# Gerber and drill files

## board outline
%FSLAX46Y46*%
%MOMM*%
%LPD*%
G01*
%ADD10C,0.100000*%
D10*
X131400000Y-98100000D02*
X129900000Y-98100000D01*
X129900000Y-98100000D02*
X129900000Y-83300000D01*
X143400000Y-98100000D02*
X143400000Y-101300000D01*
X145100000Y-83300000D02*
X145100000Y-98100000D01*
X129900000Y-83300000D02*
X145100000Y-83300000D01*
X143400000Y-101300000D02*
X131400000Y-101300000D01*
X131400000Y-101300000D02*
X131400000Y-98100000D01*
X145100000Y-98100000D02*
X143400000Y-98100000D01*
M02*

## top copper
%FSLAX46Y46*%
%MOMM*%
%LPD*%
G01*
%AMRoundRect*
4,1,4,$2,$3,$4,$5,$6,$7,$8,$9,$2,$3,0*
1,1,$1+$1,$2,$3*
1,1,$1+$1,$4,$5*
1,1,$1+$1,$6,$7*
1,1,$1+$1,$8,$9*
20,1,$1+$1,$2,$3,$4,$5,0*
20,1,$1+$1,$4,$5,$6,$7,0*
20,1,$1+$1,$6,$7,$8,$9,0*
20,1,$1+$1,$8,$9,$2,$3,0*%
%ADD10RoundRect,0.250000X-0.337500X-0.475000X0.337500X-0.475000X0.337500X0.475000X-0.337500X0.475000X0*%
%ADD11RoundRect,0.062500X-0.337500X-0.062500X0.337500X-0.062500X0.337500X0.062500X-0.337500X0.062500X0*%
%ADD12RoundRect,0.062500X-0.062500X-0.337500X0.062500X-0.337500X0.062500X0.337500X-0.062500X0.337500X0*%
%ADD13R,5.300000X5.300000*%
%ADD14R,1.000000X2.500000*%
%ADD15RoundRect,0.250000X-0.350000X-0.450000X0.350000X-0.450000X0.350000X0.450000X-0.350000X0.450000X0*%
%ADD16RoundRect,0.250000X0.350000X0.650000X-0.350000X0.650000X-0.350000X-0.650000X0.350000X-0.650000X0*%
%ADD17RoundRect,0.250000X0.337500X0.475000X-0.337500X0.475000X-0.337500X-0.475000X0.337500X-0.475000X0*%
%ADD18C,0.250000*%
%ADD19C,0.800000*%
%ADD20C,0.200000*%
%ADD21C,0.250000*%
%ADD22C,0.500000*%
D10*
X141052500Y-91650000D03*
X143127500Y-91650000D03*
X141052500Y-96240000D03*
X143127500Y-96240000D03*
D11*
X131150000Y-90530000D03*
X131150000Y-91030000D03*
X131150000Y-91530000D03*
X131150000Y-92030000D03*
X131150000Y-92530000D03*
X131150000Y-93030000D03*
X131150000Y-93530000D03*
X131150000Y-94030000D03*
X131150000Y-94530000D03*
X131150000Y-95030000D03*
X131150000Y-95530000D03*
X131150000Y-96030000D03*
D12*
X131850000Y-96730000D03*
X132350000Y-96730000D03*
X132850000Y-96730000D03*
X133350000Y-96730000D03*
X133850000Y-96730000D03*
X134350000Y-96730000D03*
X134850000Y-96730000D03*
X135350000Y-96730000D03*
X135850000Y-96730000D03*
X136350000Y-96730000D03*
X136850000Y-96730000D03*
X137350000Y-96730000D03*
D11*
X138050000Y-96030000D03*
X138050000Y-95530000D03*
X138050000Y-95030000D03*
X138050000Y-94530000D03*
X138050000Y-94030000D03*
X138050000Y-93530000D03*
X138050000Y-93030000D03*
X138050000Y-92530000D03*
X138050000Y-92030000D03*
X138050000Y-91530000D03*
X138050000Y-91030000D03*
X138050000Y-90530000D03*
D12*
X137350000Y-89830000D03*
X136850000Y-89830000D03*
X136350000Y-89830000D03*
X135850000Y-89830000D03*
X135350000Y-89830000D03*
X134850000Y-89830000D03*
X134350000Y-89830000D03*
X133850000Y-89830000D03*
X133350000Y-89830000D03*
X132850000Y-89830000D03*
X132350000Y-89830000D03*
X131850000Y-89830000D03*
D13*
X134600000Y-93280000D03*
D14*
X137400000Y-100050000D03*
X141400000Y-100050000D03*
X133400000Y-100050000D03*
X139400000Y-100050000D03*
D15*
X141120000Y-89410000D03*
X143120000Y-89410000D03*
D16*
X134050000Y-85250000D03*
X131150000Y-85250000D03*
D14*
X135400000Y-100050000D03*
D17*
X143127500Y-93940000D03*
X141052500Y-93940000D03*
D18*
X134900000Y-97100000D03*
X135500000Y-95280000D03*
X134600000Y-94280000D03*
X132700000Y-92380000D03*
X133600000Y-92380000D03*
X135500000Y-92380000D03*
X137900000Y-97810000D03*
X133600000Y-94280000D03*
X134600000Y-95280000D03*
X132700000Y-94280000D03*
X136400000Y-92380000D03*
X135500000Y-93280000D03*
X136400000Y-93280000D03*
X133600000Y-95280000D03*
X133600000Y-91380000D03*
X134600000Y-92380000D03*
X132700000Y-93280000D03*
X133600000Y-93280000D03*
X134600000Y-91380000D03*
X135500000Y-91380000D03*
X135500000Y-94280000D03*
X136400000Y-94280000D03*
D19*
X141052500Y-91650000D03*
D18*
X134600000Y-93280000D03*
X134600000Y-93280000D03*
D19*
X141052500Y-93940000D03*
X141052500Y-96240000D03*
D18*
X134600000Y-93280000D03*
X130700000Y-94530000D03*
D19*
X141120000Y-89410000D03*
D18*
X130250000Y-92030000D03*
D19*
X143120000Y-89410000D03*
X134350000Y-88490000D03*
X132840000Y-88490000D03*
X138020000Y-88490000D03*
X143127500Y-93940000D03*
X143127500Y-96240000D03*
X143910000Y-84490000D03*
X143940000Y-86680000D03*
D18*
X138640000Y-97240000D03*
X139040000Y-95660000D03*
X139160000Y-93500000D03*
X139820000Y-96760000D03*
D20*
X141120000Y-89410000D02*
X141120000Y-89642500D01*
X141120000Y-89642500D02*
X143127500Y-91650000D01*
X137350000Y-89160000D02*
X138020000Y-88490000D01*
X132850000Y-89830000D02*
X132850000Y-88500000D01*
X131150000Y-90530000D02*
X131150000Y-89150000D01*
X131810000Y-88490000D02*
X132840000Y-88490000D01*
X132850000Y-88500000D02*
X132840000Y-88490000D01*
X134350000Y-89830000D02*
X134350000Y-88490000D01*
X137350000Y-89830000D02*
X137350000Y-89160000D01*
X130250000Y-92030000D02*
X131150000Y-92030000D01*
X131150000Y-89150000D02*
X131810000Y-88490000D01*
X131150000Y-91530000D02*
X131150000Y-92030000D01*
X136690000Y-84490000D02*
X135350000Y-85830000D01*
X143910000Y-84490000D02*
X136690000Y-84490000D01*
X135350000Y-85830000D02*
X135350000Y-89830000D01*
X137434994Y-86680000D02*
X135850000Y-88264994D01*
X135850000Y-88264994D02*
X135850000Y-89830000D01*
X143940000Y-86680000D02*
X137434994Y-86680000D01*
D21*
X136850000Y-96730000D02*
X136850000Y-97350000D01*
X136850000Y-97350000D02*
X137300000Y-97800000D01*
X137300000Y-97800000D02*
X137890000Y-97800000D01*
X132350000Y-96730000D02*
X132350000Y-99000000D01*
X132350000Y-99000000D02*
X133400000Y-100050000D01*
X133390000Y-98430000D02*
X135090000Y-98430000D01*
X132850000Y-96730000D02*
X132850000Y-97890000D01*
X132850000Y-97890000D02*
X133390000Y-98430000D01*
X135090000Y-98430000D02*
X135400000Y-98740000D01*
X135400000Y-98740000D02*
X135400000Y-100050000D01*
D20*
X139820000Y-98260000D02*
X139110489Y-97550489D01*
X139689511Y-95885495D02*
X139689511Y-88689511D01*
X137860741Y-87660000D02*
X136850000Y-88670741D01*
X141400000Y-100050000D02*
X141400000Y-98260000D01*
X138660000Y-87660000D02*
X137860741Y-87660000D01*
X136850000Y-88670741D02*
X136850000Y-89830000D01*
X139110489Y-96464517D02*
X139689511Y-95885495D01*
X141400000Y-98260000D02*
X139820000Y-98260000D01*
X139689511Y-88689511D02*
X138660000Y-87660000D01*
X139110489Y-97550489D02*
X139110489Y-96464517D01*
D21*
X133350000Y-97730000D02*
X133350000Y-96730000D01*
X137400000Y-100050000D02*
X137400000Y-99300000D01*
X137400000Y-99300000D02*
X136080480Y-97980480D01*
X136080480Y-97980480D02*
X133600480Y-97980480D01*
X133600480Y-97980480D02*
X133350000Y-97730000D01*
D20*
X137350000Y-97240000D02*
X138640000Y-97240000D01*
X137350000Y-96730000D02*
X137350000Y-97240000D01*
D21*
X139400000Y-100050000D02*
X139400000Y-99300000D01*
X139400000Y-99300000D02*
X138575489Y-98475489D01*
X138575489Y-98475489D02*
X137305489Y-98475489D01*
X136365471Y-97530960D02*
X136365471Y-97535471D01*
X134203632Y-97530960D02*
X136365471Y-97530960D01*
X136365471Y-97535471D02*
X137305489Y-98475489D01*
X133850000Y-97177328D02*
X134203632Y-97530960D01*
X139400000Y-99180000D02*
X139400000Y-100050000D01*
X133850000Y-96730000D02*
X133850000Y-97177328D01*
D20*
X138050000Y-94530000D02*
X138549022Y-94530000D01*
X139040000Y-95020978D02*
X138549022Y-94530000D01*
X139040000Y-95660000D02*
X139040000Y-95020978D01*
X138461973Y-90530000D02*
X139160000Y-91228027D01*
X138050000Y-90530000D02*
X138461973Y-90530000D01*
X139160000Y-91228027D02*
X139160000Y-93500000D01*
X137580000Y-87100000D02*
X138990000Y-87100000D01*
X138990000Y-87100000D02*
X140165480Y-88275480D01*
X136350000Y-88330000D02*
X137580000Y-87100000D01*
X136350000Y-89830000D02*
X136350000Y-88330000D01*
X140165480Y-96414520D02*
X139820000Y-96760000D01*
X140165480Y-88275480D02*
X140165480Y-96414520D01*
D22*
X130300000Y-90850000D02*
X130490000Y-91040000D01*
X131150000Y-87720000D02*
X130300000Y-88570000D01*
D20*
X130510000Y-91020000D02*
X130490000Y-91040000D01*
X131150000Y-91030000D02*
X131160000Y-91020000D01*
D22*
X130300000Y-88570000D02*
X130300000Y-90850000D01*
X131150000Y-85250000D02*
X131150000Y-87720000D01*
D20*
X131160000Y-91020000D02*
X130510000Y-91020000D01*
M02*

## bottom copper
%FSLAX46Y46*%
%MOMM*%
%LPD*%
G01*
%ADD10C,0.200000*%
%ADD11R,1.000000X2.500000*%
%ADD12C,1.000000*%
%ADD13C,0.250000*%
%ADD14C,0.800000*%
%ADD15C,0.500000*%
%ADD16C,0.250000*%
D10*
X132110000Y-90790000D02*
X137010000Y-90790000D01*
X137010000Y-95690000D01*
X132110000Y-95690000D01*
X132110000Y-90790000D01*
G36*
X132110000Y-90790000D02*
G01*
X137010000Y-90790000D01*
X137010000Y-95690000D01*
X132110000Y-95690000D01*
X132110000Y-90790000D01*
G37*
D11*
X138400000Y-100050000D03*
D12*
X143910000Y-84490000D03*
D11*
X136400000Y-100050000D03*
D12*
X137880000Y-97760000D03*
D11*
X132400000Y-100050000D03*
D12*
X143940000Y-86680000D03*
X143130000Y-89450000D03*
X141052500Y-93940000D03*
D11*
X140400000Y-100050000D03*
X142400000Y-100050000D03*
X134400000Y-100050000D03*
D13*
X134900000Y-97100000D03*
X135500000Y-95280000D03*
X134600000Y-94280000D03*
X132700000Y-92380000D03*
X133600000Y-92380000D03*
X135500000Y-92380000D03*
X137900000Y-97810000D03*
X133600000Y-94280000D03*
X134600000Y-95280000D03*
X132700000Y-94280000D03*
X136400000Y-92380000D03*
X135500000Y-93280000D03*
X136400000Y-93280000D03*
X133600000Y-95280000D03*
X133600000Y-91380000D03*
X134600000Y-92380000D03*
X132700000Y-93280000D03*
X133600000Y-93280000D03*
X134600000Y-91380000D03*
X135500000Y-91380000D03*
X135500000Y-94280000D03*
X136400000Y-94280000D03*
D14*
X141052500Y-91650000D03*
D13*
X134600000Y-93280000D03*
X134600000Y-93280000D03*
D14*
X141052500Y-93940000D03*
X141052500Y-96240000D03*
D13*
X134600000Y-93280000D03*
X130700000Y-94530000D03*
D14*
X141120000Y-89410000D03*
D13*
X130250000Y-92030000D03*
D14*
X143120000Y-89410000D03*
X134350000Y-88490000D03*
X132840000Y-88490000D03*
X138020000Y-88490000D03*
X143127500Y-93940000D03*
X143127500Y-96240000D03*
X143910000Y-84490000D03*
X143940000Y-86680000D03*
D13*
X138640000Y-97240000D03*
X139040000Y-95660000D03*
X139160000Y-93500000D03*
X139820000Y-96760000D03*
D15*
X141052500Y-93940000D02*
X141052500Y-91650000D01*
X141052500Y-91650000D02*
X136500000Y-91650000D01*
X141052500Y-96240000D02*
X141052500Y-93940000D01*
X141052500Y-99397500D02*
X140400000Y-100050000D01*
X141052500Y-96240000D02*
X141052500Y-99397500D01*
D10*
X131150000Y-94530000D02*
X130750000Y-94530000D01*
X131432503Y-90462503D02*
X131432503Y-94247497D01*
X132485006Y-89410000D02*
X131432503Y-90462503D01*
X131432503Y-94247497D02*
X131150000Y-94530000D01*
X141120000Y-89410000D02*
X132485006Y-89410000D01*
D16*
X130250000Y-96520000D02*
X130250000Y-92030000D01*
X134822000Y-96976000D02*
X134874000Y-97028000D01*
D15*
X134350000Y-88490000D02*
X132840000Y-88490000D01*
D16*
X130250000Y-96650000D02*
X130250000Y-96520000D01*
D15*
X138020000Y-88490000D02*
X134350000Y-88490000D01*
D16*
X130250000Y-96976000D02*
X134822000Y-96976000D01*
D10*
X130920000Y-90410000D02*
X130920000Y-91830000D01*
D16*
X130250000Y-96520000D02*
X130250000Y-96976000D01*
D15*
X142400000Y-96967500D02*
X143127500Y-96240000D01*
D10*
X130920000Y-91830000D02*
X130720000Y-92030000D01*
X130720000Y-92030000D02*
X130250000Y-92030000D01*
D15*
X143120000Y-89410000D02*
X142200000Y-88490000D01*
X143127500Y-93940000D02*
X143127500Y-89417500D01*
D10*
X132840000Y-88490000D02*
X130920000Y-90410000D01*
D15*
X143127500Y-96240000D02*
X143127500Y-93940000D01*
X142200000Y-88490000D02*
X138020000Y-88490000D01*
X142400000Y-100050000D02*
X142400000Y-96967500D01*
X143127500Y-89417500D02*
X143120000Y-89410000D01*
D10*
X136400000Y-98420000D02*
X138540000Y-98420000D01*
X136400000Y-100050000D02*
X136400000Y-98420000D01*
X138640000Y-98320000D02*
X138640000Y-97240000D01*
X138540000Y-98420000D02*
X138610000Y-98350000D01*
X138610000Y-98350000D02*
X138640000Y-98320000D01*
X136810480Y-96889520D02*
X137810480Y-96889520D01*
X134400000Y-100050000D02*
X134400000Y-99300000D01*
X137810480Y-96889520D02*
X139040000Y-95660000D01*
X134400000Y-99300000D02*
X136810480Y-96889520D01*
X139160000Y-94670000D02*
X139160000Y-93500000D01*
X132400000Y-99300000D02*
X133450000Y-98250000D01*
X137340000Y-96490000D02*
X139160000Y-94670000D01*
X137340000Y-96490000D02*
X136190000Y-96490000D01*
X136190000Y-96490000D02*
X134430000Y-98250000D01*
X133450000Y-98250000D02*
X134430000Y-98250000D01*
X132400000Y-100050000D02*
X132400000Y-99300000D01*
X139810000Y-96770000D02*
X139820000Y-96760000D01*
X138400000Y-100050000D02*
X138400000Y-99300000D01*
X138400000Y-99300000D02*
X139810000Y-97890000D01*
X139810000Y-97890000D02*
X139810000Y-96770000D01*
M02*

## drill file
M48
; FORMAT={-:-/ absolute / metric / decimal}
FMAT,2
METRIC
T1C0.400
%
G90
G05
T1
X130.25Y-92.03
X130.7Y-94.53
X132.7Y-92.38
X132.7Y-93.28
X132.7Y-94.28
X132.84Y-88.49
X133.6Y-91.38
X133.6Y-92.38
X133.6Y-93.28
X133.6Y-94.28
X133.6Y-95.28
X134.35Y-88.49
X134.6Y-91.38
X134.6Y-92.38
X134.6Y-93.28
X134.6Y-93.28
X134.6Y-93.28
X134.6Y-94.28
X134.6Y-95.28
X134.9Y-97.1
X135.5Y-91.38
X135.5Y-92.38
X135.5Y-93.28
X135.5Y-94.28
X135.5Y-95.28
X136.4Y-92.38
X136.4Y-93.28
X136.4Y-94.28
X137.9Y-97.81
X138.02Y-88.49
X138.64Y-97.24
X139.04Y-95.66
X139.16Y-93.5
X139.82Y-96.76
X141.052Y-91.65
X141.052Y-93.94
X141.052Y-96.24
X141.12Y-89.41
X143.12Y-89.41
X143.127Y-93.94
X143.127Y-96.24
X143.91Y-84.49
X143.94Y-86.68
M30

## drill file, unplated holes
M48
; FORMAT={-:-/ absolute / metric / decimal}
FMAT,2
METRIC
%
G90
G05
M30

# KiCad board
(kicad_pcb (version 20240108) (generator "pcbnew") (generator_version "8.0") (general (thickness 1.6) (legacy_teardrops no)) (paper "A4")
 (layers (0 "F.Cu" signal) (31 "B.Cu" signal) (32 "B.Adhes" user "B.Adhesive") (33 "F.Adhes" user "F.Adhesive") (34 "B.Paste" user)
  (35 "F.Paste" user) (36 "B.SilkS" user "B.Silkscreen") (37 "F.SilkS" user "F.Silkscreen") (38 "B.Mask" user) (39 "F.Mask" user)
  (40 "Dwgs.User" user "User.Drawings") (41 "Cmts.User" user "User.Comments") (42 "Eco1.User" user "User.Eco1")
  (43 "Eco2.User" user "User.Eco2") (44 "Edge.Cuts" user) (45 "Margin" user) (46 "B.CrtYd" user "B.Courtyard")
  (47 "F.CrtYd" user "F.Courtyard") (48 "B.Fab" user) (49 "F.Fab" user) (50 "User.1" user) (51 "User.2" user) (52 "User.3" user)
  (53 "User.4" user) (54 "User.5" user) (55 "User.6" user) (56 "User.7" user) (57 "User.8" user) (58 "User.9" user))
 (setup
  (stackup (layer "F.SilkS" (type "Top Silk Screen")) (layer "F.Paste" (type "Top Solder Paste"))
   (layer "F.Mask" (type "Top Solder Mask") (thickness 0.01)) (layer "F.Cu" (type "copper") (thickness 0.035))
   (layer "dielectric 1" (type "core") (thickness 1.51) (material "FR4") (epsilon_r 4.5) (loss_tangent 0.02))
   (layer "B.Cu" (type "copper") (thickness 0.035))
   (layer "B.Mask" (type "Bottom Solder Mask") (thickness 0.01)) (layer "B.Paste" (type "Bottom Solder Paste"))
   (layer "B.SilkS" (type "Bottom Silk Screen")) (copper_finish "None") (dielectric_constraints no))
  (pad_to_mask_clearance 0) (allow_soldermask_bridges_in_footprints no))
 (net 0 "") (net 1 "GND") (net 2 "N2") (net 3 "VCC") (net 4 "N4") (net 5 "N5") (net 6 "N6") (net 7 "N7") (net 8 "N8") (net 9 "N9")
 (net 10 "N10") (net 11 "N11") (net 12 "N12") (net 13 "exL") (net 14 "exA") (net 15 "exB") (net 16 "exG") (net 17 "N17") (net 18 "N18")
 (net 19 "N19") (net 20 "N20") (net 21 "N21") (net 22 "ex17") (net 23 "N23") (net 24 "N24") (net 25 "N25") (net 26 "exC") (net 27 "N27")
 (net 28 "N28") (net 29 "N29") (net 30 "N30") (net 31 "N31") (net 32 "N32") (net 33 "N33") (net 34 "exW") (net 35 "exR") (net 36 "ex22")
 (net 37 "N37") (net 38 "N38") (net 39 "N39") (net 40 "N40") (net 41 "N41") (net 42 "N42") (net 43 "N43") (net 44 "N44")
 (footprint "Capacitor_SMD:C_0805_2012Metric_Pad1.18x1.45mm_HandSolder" (layer "F.Cu") (at 142.09 91.65)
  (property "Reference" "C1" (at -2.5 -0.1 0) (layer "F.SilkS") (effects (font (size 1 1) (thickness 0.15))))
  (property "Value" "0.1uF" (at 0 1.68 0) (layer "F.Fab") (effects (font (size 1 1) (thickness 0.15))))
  (pad "1" smd roundrect (at -1.0375 0) (size 1.175 1.45) (layers "F.Cu" "F.Paste" "F.Mask") (roundrect_rratio 0.2127659574) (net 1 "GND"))
  (pad "2" smd roundrect (at 1.0375 0) (size 1.175 1.45) (layers "F.Cu" "F.Paste" "F.Mask") (roundrect_rratio 0.2127659574) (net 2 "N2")))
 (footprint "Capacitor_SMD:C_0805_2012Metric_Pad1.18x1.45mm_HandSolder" (layer "F.Cu") (at 142.09 96.24)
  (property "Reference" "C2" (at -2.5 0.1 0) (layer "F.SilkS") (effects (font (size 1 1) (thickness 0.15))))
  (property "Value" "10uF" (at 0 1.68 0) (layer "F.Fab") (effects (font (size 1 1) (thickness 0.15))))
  (pad "1" smd roundrect (at -1.0375 0) (size 1.175 1.45) (layers "F.Cu" "F.Paste" "F.Mask") (roundrect_rratio 0.2127659574) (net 1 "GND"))
  (pad "2" smd roundrect (at 1.0375 0) (size 1.175 1.45) (layers "F.Cu" "F.Paste" "F.Mask") (roundrect_rratio 0.2127659574) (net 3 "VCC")))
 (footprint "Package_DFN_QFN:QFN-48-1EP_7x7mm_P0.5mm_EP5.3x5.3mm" (layer "F.Cu") (at 134.6 93.28)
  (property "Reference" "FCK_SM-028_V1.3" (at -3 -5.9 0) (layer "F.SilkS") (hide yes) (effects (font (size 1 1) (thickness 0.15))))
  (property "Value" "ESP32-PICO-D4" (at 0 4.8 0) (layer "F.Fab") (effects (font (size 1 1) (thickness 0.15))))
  (pad "" smd roundrect (at -1.98 -1.98) (size 1.07 1.07) (layers "F.Paste") (roundrect_rratio 0.2336448598))
  (pad "" smd roundrect (at -1.98 -0.66) (size 1.07 1.07) (layers "F.Paste") (roundrect_rratio 0.2336448598))
  (pad "" smd roundrect (at -1.98 0.66) (size 1.07 1.07) (layers "F.Paste") (roundrect_rratio 0.2336448598))
  (pad "" smd roundrect (at -1.98 1.98) (size 1.07 1.07) (layers "F.Paste") (roundrect_rratio 0.2336448598))
  (pad "" smd roundrect (at -0.66 -1.98) (size 1.07 1.07) (layers "F.Paste") (roundrect_rratio 0.2336448598))
  (pad "" smd roundrect (at -0.66 -0.66) (size 1.07 1.07) (layers "F.Paste") (roundrect_rratio 0.2336448598))
  (pad "" smd roundrect (at -0.66 0.66) (size 1.07 1.07) (layers "F.Paste") (roundrect_rratio 0.2336448598))
  (pad "" smd roundrect (at -0.66 1.98) (size 1.07 1.07) (layers "F.Paste") (roundrect_rratio 0.2336448598))
  (pad "" smd roundrect (at 0.66 -1.98) (size 1.07 1.07) (layers "F.Paste") (roundrect_rratio 0.2336448598))
  (pad "" smd roundrect (at 0.66 -0.66) (size 1.07 1.07) (layers "F.Paste") (roundrect_rratio 0.2336448598))
  (pad "" smd roundrect (at 0.66 0.66) (size 1.07 1.07) (layers "F.Paste") (roundrect_rratio 0.2336448598))
  (pad "" smd roundrect (at 0.66 1.98) (size 1.07 1.07) (layers "F.Paste") (roundrect_rratio 0.2336448598))
  (pad "" smd roundrect (at 1.98 -1.98) (size 1.07 1.07) (layers "F.Paste") (roundrect_rratio 0.2336448598))
  (pad "" smd roundrect (at 1.98 -0.66) (size 1.07 1.07) (layers "F.Paste") (roundrect_rratio 0.2336448598))
  (pad "" smd roundrect (at 1.98 0.66) (size 1.07 1.07) (layers "F.Paste") (roundrect_rratio 0.2336448598))
  (pad "" smd roundrect (at 1.98 1.98) (size 1.07 1.07) (layers "F.Paste") (roundrect_rratio 0.2336448598))
  (pad "1" smd roundrect (at -3.45 -2.75) (size 0.8 0.25) (layers "F.Cu" "F.Paste" "F.Mask") (roundrect_rratio 0.25) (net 3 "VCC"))
  (pad "2" smd roundrect (at -3.45 -2.25) (size 0.8 0.25) (layers "F.Cu" "F.Paste" "F.Mask") (roundrect_rratio 0.25) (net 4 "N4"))
  (pad "3" smd roundrect (at -3.45 -1.75) (size 0.8 0.25) (layers "F.Cu" "F.Paste" "F.Mask") (roundrect_rratio 0.25) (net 3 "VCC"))
  (pad "4" smd roundrect (at -3.45 -1.25) (size 0.8 0.25) (layers "F.Cu" "F.Paste" "F.Mask") (roundrect_rratio 0.25) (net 3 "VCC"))
  (pad "5" smd roundrect (at -3.45 -0.75) (size 0.8 0.25) (layers "F.Cu" "F.Paste" "F.Mask") (roundrect_rratio 0.25) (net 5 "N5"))
  (pad "6" smd roundrect (at -3.45 -0.25) (size 0.8 0.25) (layers "F.Cu" "F.Paste" "F.Mask") (roundrect_rratio 0.25) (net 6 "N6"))
  (pad "7" smd roundrect (at -3.45 0.25) (size 0.8 0.25) (layers "F.Cu" "F.Paste" "F.Mask") (roundrect_rratio 0.25) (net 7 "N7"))
  (pad "8" smd roundrect (at -3.45 0.75) (size 0.8 0.25) (layers "F.Cu" "F.Paste" "F.Mask") (roundrect_rratio 0.25) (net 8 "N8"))
  (pad "9" smd roundrect (at -3.45 1.25) (size 0.8 0.25) (layers "F.Cu" "F.Paste" "F.Mask") (roundrect_rratio 0.25) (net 2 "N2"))
  (pad "10" smd roundrect (at -3.45 1.75) (size 0.8 0.25) (layers "F.Cu" "F.Paste" "F.Mask") (roundrect_rratio 0.25) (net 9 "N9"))
  (pad "11" smd roundrect (at -3.45 2.25) (size 0.8 0.25) (layers "F.Cu" "F.Paste" "F.Mask") (roundrect_rratio 0.25) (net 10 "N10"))
  (pad "12" smd roundrect (at -3.45 2.75) (size 0.8 0.25) (layers "F.Cu" "F.Paste" "F.Mask") (roundrect_rratio 0.25) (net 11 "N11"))
  (pad "13" smd roundrect (at -2.75 3.45) (size 0.25 0.8) (layers "F.Cu" "F.Paste" "F.Mask") (roundrect_rratio 0.25) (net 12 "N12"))
  (pad "14" smd roundrect (at -2.25 3.45) (size 0.25 0.8) (layers "F.Cu" "F.Paste" "F.Mask") (roundrect_rratio 0.25) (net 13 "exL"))
  (pad "15" smd roundrect (at -1.75 3.45) (size 0.25 0.8) (layers "F.Cu" "F.Paste" "F.Mask") (roundrect_rratio 0.25) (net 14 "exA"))
  (pad "16" smd roundrect (at -1.25 3.45) (size 0.25 0.8) (layers "F.Cu" "F.Paste" "F.Mask") (roundrect_rratio 0.25) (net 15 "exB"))
  (pad "17" smd roundrect (at -0.75 3.45) (size 0.25 0.8) (layers "F.Cu" "F.Paste" "F.Mask") (roundrect_rratio 0.25) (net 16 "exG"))
  (pad "18" smd roundrect (at -0.25 3.45) (size 0.25 0.8) (layers "F.Cu" "F.Paste" "F.Mask") (roundrect_rratio 0.25) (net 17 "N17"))
  (pad "19" smd roundrect (at 0.25 3.45) (size 0.25 0.8) (layers "F.Cu" "F.Paste" "F.Mask") (roundrect_rratio 0.25) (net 3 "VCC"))
  (pad "20" smd roundrect (at 0.75 3.45) (size 0.25 0.8) (layers "F.Cu" "F.Paste" "F.Mask") (roundrect_rratio 0.25) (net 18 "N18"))
  (pad "21" smd roundrect (at 1.25 3.45) (size 0.25 0.8) (layers "F.Cu" "F.Paste" "F.Mask") (roundrect_rratio 0.25) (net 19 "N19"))
  (pad "22" smd roundrect (at 1.75 3.45) (size 0.25 0.8) (layers "F.Cu" "F.Paste" "F.Mask") (roundrect_rratio 0.25) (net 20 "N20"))
  (pad "23" smd roundrect (at 2.25 3.45) (size 0.25 0.8) (layers "F.Cu" "F.Paste" "F.Mask") (roundrect_rratio 0.25) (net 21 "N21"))
  (pad "24" smd roundrect (at 2.75 3.45) (size 0.25 0.8) (layers "F.Cu" "F.Paste" "F.Mask") (roundrect_rratio 0.25) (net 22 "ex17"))
  (pad "25" smd roundrect (at 3.45 2.75) (size 0.8 0.25) (layers "F.Cu" "F.Paste" "F.Mask") (roundrect_rratio 0.25) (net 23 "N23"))
  (pad "26" smd roundrect (at 3.45 2.25) (size 0.8 0.25) (layers "F.Cu" "F.Paste" "F.Mask") (roundrect_rratio 0.25) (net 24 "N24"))
  (pad "27" smd roundrect (at 3.45 1.75) (size 0.8 0.25) (layers "F.Cu" "F.Paste" "F.Mask") (roundrect_rratio 0.25) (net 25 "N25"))
  (pad "28" smd roundrect (at 3.45 1.25) (size 0.8 0.25) (layers "F.Cu" "F.Paste" "F.Mask") (roundrect_rratio 0.25) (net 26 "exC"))
  (pad "29" smd roundrect (at 3.45 0.75) (size 0.8 0.25) (layers "F.Cu" "F.Paste" "F.Mask") (roundrect_rratio 0.25) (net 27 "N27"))
  (pad "30" smd roundrect (at 3.45 0.25) (size 0.8 0.25) (layers "F.Cu" "F.Paste" "F.Mask") (roundrect_rratio 0.25) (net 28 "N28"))
  (pad "31" smd roundrect (at 3.45 -0.25) (size 0.8 0.25) (layers "F.Cu" "F.Paste" "F.Mask") (roundrect_rratio 0.25) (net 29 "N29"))
  (pad "32" smd roundrect (at 3.45 -0.75) (size 0.8 0.25) (layers "F.Cu" "F.Paste" "F.Mask") (roundrect_rratio 0.25) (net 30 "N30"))
  (pad "33" smd roundrect (at 3.45 -1.25) (size 0.8 0.25) (layers "F.Cu" "F.Paste" "F.Mask") (roundrect_rratio 0.25) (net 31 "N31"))
  (pad "34" smd roundrect (at 3.45 -1.75) (size 0.8 0.25) (layers "F.Cu" "F.Paste" "F.Mask") (roundrect_rratio 0.25) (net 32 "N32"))
  (pad "35" smd roundrect (at 3.45 -2.25) (size 0.8 0.25) (layers "F.Cu" "F.Paste" "F.Mask") (roundrect_rratio 0.25) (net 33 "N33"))
  (pad "36" smd roundrect (at 3.45 -2.75) (size 0.8 0.25) (layers "F.Cu" "F.Paste" "F.Mask") (roundrect_rratio 0.25) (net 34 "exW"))
  (pad "37" smd roundrect (at 2.75 -3.45) (size 0.25 0.8) (layers "F.Cu" "F.Paste" "F.Mask") (roundrect_rratio 0.25) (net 3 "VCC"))
  (pad "38" smd roundrect (at 2.25 -3.45) (size 0.25 0.8) (layers "F.Cu" "F.Paste" "F.Mask") (roundrect_rratio 0.25) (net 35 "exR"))
  (pad "39" smd roundrect (at 1.75 -3.45) (size 0.25 0.8) (layers "F.Cu" "F.Paste" "F.Mask") (roundrect_rratio 0.25) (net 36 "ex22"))
  (pad "40" smd roundrect (at 1.25 -3.45) (size 0.25 0.8) (layers "F.Cu" "F.Paste" "F.Mask") (roundrect_rratio 0.25) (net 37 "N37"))
  (pad "41" smd roundrect (at 0.75 -3.45) (size 0.25 0.8) (layers "F.Cu" "F.Paste" "F.Mask") (roundrect_rratio 0.25) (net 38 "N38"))
  (pad "42" smd roundrect (at 0.25 -3.45) (size 0.25 0.8) (layers "F.Cu" "F.Paste" "F.Mask") (roundrect_rratio 0.25) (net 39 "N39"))
  (pad "43" smd roundrect (at -0.25 -3.45) (size 0.25 0.8) (layers "F.Cu" "F.Paste" "F.Mask") (roundrect_rratio 0.25) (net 3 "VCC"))
  (pad "44" smd roundrect (at -0.75 -3.45) (size 0.25 0.8) (layers "F.Cu" "F.Paste" "F.Mask") (roundrect_rratio 0.25) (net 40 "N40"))
  (pad "45" smd roundrect (at -1.25 -3.45) (size 0.25 0.8) (layers "F.Cu" "F.Paste" "F.Mask") (roundrect_rratio 0.25) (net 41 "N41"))
  (pad "46" smd roundrect (at -1.75 -3.45) (size 0.25 0.8) (layers "F.Cu" "F.Paste" "F.Mask") (roundrect_rratio 0.25) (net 3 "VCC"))
  (pad "47" smd roundrect (at -2.25 -3.45) (size 0.25 0.8) (layers "F.Cu" "F.Paste" "F.Mask") (roundrect_rratio 0.25) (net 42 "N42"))
  (pad "48" smd roundrect (at -2.75 -3.45) (size 0.25 0.8) (layers "F.Cu" "F.Paste" "F.Mask") (roundrect_rratio 0.25) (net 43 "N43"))
  (pad "49" smd rect (at 0 0) (size 5.3 5.3) (layers "F.Cu" "F.Mask") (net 1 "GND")))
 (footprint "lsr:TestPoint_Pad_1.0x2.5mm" (layer "F.Cu") (at 137.4 100.85 90)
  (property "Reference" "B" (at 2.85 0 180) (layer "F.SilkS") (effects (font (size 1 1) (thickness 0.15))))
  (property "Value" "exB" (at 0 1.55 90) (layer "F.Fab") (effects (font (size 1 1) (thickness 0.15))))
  (pad "1" smd rect (at 0.8 0 90) (size 2.5 1) (layers "F.Cu" "F.Mask") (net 15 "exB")))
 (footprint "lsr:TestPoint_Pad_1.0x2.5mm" (layer "F.Cu") (at 141.4 100.8 90)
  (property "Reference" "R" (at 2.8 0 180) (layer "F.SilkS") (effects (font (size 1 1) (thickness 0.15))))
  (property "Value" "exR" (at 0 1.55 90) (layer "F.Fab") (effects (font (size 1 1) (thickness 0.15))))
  (pad "1" smd rect (at 0.75 0 90) (size 2.5 1) (layers "F.Cu" "F.Mask") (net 35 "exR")))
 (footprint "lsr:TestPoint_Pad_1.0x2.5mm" (layer "F.Cu") (at 133.4 100.8 90)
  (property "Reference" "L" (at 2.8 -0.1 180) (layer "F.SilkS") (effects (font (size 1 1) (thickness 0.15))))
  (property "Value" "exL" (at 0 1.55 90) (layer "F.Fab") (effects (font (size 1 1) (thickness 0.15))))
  (pad "1" smd rect (at 0.75 0 90) (size 2.5 1) (layers "F.Cu" "F.Mask") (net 13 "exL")))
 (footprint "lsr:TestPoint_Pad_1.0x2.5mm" (layer "F.Cu") (at 139.4 100.75 90)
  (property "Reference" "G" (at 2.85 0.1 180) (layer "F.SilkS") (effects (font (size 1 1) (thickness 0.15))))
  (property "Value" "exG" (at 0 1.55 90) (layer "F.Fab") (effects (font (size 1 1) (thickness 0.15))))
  (pad "1" smd rect (at 0.7 0 90) (size 2.5 1) (layers "F.Cu" "F.Mask") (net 16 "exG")))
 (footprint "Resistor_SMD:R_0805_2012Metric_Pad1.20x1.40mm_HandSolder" (layer "F.Cu") (at 142.12 89.41)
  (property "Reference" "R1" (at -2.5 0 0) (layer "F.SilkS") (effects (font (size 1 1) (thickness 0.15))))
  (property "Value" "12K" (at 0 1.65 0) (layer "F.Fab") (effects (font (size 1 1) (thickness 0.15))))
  (pad "1" smd roundrect (at -1 0) (size 1.2 1.4) (layers "F.Cu" "F.Paste" "F.Mask") (roundrect_rratio 0.2083333333) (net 2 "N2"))
  (pad "2" smd roundrect (at 1 0) (size 1.2 1.4) (layers "F.Cu" "F.Paste" "F.Mask") (roundrect_rratio 0.2083333333) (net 3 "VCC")))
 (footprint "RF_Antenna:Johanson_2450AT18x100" (layer "F.Cu") (at 132.6 85.25 180)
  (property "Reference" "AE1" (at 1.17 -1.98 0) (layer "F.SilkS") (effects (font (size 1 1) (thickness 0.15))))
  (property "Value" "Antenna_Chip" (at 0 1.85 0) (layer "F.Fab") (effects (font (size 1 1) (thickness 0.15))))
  (pad "1" smd roundrect (at -1.45 0 180) (size 1.2 1.8) (layers "F.Cu" "F.Paste" "F.Mask") (roundrect_rratio 0.2083333333) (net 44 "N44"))
  (pad "2" smd roundrect (at 1.45 0 180) (size 1.2 1.8) (layers "F.Cu" "F.Paste" "F.Mask") (roundrect_rratio 0.2083333333) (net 4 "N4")))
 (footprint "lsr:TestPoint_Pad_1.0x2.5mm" (layer "F.Cu") (at 135.4 100.8 90)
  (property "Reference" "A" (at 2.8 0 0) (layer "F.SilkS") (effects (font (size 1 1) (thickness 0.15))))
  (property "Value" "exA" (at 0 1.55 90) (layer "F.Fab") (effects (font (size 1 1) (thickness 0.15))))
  (pad "1" smd rect (at 0.75 0 90) (size 2.5 1) (layers "F.Cu" "F.Mask") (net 14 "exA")))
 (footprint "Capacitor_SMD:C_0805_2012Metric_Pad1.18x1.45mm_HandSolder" (layer "F.Cu") (at 142.09 93.94 180)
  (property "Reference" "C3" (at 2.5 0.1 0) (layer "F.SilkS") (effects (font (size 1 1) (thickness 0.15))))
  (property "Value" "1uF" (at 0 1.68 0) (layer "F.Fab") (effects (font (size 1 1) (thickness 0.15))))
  (pad "1" smd roundrect (at -1.0375 0 180) (size 1.175 1.45) (layers "F.Cu" "F.Paste" "F.Mask") (roundrect_rratio 0.2127659574)
   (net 3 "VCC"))
  (pad "2" smd roundrect (at 1.0375 0 180) (size 1.175 1.45) (layers "F.Cu" "F.Paste" "F.Mask") (roundrect_rratio 0.2127659574)
   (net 1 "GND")))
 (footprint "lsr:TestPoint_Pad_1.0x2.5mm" (layer "B.Cu") (at 138.4 100.75 90)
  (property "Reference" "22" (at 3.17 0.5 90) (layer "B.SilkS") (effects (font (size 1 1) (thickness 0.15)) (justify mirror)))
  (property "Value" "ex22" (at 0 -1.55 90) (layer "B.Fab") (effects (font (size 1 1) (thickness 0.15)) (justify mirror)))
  (pad "1" smd rect (at 0.7 0 90) (size 2.5 1) (layers "B.Cu" "B.Mask") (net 36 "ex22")))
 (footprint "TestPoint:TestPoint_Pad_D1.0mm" (layer "B.Cu") (at 143.91 84.49 180)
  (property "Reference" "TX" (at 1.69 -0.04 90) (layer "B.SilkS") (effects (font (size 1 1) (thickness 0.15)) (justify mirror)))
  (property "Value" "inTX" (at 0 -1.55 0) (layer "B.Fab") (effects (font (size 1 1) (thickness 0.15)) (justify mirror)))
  (pad "1" smd circle (at 0 0 180) (size 1 1) (layers "B.Cu" "B.Mask") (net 38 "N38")))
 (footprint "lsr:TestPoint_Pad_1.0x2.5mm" (layer "B.Cu") (at 136.4 99.3 -90)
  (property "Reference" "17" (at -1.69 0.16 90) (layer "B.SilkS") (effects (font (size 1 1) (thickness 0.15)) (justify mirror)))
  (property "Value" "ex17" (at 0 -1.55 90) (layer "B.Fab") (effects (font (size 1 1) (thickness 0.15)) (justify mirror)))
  (pad "1" smd rect (at 0.75 0 270) (size 2.5 1) (layers "B.Cu" "B.Mask") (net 22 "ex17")))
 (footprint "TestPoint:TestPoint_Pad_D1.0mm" (layer "B.Cu") (at 137.88 97.76 180)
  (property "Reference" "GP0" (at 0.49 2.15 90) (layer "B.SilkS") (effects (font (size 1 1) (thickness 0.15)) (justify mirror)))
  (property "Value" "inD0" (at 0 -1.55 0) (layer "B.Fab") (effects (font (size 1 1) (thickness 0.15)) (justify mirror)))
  (pad "1" smd circle (at 0 0 180) (size 1 1) (layers "B.Cu" "B.Mask")))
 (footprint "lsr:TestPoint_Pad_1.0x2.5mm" (layer "B.Cu") (at 132.4 100.9 90)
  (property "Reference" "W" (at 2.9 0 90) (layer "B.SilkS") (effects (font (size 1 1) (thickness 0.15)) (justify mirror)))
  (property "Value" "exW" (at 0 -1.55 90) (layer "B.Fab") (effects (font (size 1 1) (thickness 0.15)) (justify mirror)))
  (pad "1" smd rect (at 0.85 0 90) (size 2.5 1) (layers "B.Cu" "B.Mask") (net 34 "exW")))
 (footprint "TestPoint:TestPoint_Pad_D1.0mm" (layer "B.Cu") (at 143.94 86.68 180)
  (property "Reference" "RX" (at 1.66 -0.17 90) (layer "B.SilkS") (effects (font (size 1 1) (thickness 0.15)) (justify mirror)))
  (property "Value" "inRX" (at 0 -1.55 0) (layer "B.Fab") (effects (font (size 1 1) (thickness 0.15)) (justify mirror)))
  (pad "1" smd circle (at 0 0 180) (size 1 1) (layers "B.Cu" "B.Mask") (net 37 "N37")))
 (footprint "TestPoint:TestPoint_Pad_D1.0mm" (layer "B.Cu") (at 143.13 89.45 180)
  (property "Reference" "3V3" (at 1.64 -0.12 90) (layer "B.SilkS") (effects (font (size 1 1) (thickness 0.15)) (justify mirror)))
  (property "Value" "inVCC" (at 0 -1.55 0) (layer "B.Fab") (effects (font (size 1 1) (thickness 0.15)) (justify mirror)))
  (pad "1" smd circle (at 0 0 180) (size 1 1) (layers "B.Cu" "B.Mask") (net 3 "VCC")))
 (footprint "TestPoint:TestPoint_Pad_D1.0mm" (layer "B.Cu") (at 141.0525 93.94 180)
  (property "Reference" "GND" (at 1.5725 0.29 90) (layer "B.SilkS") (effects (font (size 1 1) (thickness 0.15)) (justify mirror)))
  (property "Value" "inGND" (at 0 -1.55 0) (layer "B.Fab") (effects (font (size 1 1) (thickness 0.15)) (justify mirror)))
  (pad "1" smd circle (at 0 0 180) (size 1 1) (layers "B.Cu" "B.Mask") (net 1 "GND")))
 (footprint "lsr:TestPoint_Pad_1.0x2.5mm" (layer "B.Cu") (at 140.4 99.3 -90)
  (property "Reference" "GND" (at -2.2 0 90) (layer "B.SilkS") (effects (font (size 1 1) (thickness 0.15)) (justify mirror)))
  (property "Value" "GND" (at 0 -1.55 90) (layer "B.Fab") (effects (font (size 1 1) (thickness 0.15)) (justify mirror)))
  (pad "1" smd rect (at 0.75 0 270) (size 2.5 1) (layers "B.Cu" "B.Mask") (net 1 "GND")))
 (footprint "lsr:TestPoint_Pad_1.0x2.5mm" (layer "B.Cu") (at 142.4 99.3 -90)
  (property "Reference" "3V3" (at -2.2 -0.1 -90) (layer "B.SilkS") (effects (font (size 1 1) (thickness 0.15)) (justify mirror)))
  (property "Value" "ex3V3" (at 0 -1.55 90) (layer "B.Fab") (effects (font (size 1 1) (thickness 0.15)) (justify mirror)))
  (pad "1" smd rect (at 0.75 0 270) (size 2.5 1) (layers "B.Cu" "B.Mask") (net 3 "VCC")))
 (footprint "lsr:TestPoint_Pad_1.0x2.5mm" (layer "B.Cu") (at 134.4 99.3 -90)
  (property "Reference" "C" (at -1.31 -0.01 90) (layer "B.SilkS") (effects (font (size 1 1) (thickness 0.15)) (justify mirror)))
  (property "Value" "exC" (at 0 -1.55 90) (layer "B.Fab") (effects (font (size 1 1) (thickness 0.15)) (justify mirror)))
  (pad "1" smd rect (at 0.75 0 270) (size 2.5 1) (layers "B.Cu" "B.Mask") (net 26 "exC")))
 (gr_rect (start 132.11 90.79) (end 137.01 95.69) (stroke (width 0.2) (type solid)) (fill solid) (layer "B.Cu") (net 1))
 (gr_line (start 131.4 98.1) (end 129.9 98.1) (stroke (width 0.1) (type solid)) (layer "Edge.Cuts"))
 (gr_line (start 129.9 98.1) (end 129.9 83.3) (stroke (width 0.1) (type solid)) (layer "Edge.Cuts"))
 (gr_line (start 143.4 98.1) (end 143.4 101.3) (stroke (width 0.1) (type solid)) (layer "Edge.Cuts"))
 (gr_line (start 145.1 83.3) (end 145.1 98.1) (stroke (width 0.1) (type solid)) (layer "Edge.Cuts"))
 (gr_line (start 129.9 83.3) (end 145.1 83.3) (stroke (width 0.1) (type solid)) (layer "Edge.Cuts"))
 (gr_line (start 143.4 101.3) (end 131.4 101.3) (stroke (width 0.1) (type solid)) (layer "Edge.Cuts"))
 (gr_line (start 131.4 101.3) (end 131.4 98.1) (stroke (width 0.1) (type solid)) (layer "Edge.Cuts"))
 (gr_line (start 145.1 98.1) (end 143.4 98.1) (stroke (width 0.1) (type solid)) (layer "Edge.Cuts"))
 (via (at 135.5 95.28) (size 0.25) (drill 0.4) (layers "F.Cu" "B.Cu") (free yes) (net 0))
 (via (at 134.6 94.28) (size 0.25) (drill 0.4) (layers "F.Cu" "B.Cu") (free yes) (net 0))
 (via (at 132.7 92.38) (size 0.25) (drill 0.4) (layers "F.Cu" "B.Cu") (free yes) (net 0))
 (via (at 133.6 92.38) (size 0.25) (drill 0.4) (layers "F.Cu" "B.Cu") (free yes) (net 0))
 (via (at 135.5 92.38) (size 0.25) (drill 0.4) (layers "F.Cu" "B.Cu") (free yes) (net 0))
 (via (at 137.9 97.81) (size 0.25) (drill 0.4) (layers "F.Cu" "B.Cu") (free yes) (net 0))
 (via (at 133.6 94.28) (size 0.25) (drill 0.4) (layers "F.Cu" "B.Cu") (free yes) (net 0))
 (via (at 134.6 95.28) (size 0.25) (drill 0.4) (layers "F.Cu" "B.Cu") (free yes) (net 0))
 (via (at 132.7 94.28) (size 0.25) (drill 0.4) (layers "F.Cu" "B.Cu") (free yes) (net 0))
 (via (at 136.4 92.38) (size 0.25) (drill 0.4) (layers "F.Cu" "B.Cu") (free yes) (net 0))
 (via (at 135.5 93.28) (size 0.25) (drill 0.4) (layers "F.Cu" "B.Cu") (free yes) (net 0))
 (via (at 136.4 93.28) (size 0.25) (drill 0.4) (layers "F.Cu" "B.Cu") (free yes) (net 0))
 (via (at 133.6 95.28) (size 0.25) (drill 0.4) (layers "F.Cu" "B.Cu") (free yes) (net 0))
 (via (at 133.6 91.38) (size 0.25) (drill 0.4) (layers "F.Cu" "B.Cu") (free yes) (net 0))
 (via (at 134.6 92.38) (size 0.25) (drill 0.4) (layers "F.Cu" "B.Cu") (free yes) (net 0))
 (via (at 132.7 93.28) (size 0.25) (drill 0.4) (layers "F.Cu" "B.Cu") (free yes) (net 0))
 (via (at 133.6 93.28) (size 0.25) (drill 0.4) (layers "F.Cu" "B.Cu") (free yes) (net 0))
 (via (at 134.6 91.38) (size 0.25) (drill 0.4) (layers "F.Cu" "B.Cu") (free yes) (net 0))
 (via (at 135.5 91.38) (size 0.25) (drill 0.4) (layers "F.Cu" "B.Cu") (free yes) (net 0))
 (via (at 135.5 94.28) (size 0.25) (drill 0.4) (layers "F.Cu" "B.Cu") (free yes) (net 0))
 (via (at 136.4 94.28) (size 0.25) (drill 0.4) (layers "F.Cu" "B.Cu") (free yes) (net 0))
 (via (at 141.0525 91.65) (size 0.8) (drill 0.4) (layers "F.Cu" "B.Cu") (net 1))
 (via (at 134.6 93.28) (size 0.25) (drill 0.4) (layers "F.Cu" "B.Cu") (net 1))
 (via (at 134.6 93.28) (size 0.25) (drill 0.4) (layers "F.Cu" "B.Cu") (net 1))
 (via (at 141.0525 93.94) (size 0.8) (drill 0.4) (layers "F.Cu" "B.Cu") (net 1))
 (via (at 141.0525 96.24) (size 0.8) (drill 0.4) (layers "F.Cu" "B.Cu") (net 1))
 (via (at 134.6 93.28) (size 0.25) (drill 0.4) (layers "F.Cu" "B.Cu") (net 1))
 (segment (start 141.0525 93.94) (end 141.0525 91.65) (width 0.5) (layer "B.Cu") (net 1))
 (segment (start 141.0525 91.65) (end 136.5 91.65) (width 0.5) (layer "B.Cu") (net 1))
 (segment (start 141.0525 96.24) (end 141.0525 93.94) (width 0.5) (layer "B.Cu") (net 1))
 (segment (start 141.0525 99.3975) (end 140.4 100.05) (width 0.5) (layer "B.Cu") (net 1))
 (segment (start 141.0525 96.24) (end 141.0525 99.3975) (width 0.5) (layer "B.Cu") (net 1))
 (segment (start 141.12 89.41) (end 141.12 89.6425) (width 0.2) (layer "F.Cu") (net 2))
 (segment (start 141.12 89.6425) (end 143.1275 91.65) (width 0.2) (layer "F.Cu") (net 2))
 (via (at 130.7 94.53) (size 0.25) (drill 0.4) (layers "F.Cu" "B.Cu") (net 2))
 (via (at 141.12 89.41) (size 0.8) (drill 0.4) (layers "F.Cu" "B.Cu") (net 2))
 (segment (start 131.15 94.53) (end 130.75 94.53) (width 0.2) (layer "B.Cu") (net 2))
 (segment (start 131.432503 90.462503) (end 131.432503 94.247497) (width 0.2) (layer "B.Cu") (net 2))
 (segment (start 132.485006 89.41) (end 131.432503 90.462503) (width 0.2) (layer "B.Cu") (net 2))
 (segment (start 131.432503 94.247497) (end 131.15 94.53) (width 0.2) (layer "B.Cu") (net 2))
 (segment (start 141.12 89.41) (end 132.485006 89.41) (width 0.2) (layer "B.Cu") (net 2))
 (segment (start 137.35 89.16) (end 138.02 88.49) (width 0.2) (layer "F.Cu") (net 3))
 (segment (start 132.85 89.83) (end 132.85 88.5) (width 0.2) (layer "F.Cu") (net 3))
 (segment (start 131.15 90.53) (end 131.15 89.15) (width 0.2) (layer "F.Cu") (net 3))
 (segment (start 131.81 88.49) (end 132.84 88.49) (width 0.2) (layer "F.Cu") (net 3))
 (segment (start 132.85 88.5) (end 132.84 88.49) (width 0.2) (layer "F.Cu") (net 3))
 (segment (start 134.35 89.83) (end 134.35 88.49) (width 0.2) (layer "F.Cu") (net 3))
 (segment (start 137.35 89.83) (end 137.35 89.16) (width 0.2) (layer "F.Cu") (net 3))
 (segment (start 130.25 92.03) (end 131.15 92.03) (width 0.2) (layer "F.Cu") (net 3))
 (segment (start 131.15 89.15) (end 131.81 88.49) (width 0.2) (layer "F.Cu") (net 3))
 (segment (start 131.15 91.53) (end 131.15 92.03) (width 0.2) (layer "F.Cu") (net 3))
 (via (at 130.25 92.03) (size 0.25) (drill 0.4) (layers "F.Cu" "B.Cu") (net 3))
 (via (at 143.12 89.41) (size 0.8) (drill 0.4) (layers "F.Cu" "B.Cu") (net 3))
 (via (at 134.35 88.49) (size 0.8) (drill 0.4) (layers "F.Cu" "B.Cu") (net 3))
 (via (at 132.84 88.49) (size 0.8) (drill 0.4) (layers "F.Cu" "B.Cu") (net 3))
 (via (at 138.02 88.49) (size 0.8) (drill 0.4) (layers "F.Cu" "B.Cu") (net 3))
 (via (at 134.9 97.1) (size 0.25) (drill 0.4) (layers "F.Cu" "B.Cu") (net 3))
 (via (at 143.1275 93.94) (size 0.8) (drill 0.4) (layers "F.Cu" "B.Cu") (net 3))
 (via (at 143.1275 96.24) (size 0.8) (drill 0.4) (layers "F.Cu" "B.Cu") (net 3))
 (segment (start 130.25 96.52) (end 130.25 92.03) (width 0.25) (layer "B.Cu") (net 3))
 (segment (start 134.822 96.976) (end 134.874 97.028) (width 0.25) (layer "B.Cu") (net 3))
 (segment (start 134.35 88.49) (end 132.84 88.49) (width 0.5) (layer "B.Cu") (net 3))
 (segment (start 130.25 96.65) (end 130.25 96.52) (width 0.25) (layer "B.Cu") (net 3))
 (segment (start 138.02 88.49) (end 134.35 88.49) (width 0.5) (layer "B.Cu") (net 3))
 (segment (start 130.25 96.976) (end 134.822 96.976) (width 0.25) (layer "B.Cu") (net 3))
 (segment (start 130.92 90.41) (end 130.92 91.83) (width 0.2) (layer "B.Cu") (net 3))
 (segment (start 130.25 96.52) (end 130.25 96.976) (width 0.25) (layer "B.Cu") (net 3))
 (segment (start 142.4 96.9675) (end 143.1275 96.24) (width 0.5) (layer "B.Cu") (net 3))
 (segment (start 130.92 91.83) (end 130.72 92.03) (width 0.2) (layer "B.Cu") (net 3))
 (segment (start 130.72 92.03) (end 130.25 92.03) (width 0.2) (layer "B.Cu") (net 3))
 (segment (start 143.12 89.41) (end 142.2 88.49) (width 0.5) (layer "B.Cu") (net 3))
 (segment (start 143.1275 93.94) (end 143.1275 89.4175) (width 0.5) (layer "B.Cu") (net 3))
 (segment (start 132.84 88.49) (end 130.92 90.41) (width 0.2) (layer "B.Cu") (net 3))
 (segment (start 143.1275 96.24) (end 143.1275 93.94) (width 0.5) (layer "B.Cu") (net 3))
 (segment (start 142.2 88.49) (end 138.02 88.49) (width 0.5) (layer "B.Cu") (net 3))
 (segment (start 142.4 100.05) (end 142.4 96.9675) (width 0.5) (layer "B.Cu") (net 3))
 (segment (start 143.1275 89.4175) (end 143.12 89.41) (width 0.5) (layer "B.Cu") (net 3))
 (segment (start 136.69 84.49) (end 135.35 85.83) (width 0.2) (layer "F.Cu") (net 38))
 (segment (start 143.91 84.49) (end 136.69 84.49) (width 0.2) (layer "F.Cu") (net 38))
 (segment (start 135.35 85.83) (end 135.35 89.83) (width 0.2) (layer "F.Cu") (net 38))
 (via (at 143.91 84.49) (size 0.8) (drill 0.4) (layers "F.Cu" "B.Cu") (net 38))
 (segment (start 137.434994 86.68) (end 135.85 88.264994) (width 0.2) (layer "F.Cu") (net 37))
 (segment (start 135.85 88.264994) (end 135.85 89.83) (width 0.2) (layer "F.Cu") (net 37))
 (segment (start 143.94 86.68) (end 137.434994 86.68) (width 0.2) (layer "F.Cu") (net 37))
 (via (at 143.94 86.68) (size 0.8) (drill 0.4) (layers "F.Cu" "B.Cu") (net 37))
 (segment (start 136.85 96.73) (end 136.85 97.35) (width 0.25) (layer "F.Cu") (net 21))
 (segment (start 136.85 97.35) (end 137.3 97.8) (width 0.25) (layer "F.Cu") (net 21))
 (segment (start 137.3 97.8) (end 137.89 97.8) (width 0.25) (layer "F.Cu") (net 21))
 (segment (start 132.35 96.73) (end 132.35 99) (width 0.25) (layer "F.Cu") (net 13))
 (segment (start 132.35 99) (end 133.4 100.05) (width 0.25) (layer "F.Cu") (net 13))
 (segment (start 133.39 98.43) (end 135.09 98.43) (width 0.25) (layer "F.Cu") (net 14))
 (segment (start 132.85 96.73) (end 132.85 97.89) (width 0.25) (layer "F.Cu") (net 14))
 (segment (start 132.85 97.89) (end 133.39 98.43) (width 0.25) (layer "F.Cu") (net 14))
 (segment (start 135.09 98.43) (end 135.4 98.74) (width 0.25) (layer "F.Cu") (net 14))
 (segment (start 135.4 98.74) (end 135.4 100.05) (width 0.25) (layer "F.Cu") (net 14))
 (segment (start 139.82 98.26) (end 139.110489 97.550489) (width 0.2) (layer "F.Cu") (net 35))
 (segment (start 139.689511 95.885495) (end 139.689511 88.689511) (width 0.2) (layer "F.Cu") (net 35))
 (segment (start 137.860741 87.66) (end 136.85 88.670741) (width 0.2) (layer "F.Cu") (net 35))
 (segment (start 141.4 100.05) (end 141.4 98.26) (width 0.2) (layer "F.Cu") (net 35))
 (segment (start 138.66 87.66) (end 137.860741 87.66) (width 0.2) (layer "F.Cu") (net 35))
 (segment (start 136.85 88.670741) (end 136.85 89.83) (width 0.2) (layer "F.Cu") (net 35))
 (segment (start 139.110489 96.464517) (end 139.689511 95.885495) (width 0.2) (layer "F.Cu") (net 35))
 (segment (start 141.4 98.26) (end 139.82 98.26) (width 0.2) (layer "F.Cu") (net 35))
 (segment (start 139.689511 88.689511) (end 138.66 87.66) (width 0.2) (layer "F.Cu") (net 35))
 (segment (start 139.110489 97.550489) (end 139.110489 96.464517) (width 0.2) (layer "F.Cu") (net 35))
 (segment (start 133.35 97.73) (end 133.35 96.73) (width 0.25) (layer "F.Cu") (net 15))
 (segment (start 137.4 100.05) (end 137.4 99.3) (width 0.25) (layer "F.Cu") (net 15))
 (segment (start 137.4 99.3) (end 136.08048 97.98048) (width 0.25) (layer "F.Cu") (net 15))
 (segment (start 136.08048 97.98048) (end 133.60048 97.98048) (width 0.25) (layer "F.Cu") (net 15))
 (segment (start 133.60048 97.98048) (end 133.35 97.73) (width 0.25) (layer "F.Cu") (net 15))
 (segment (start 137.35 97.24) (end 138.64 97.24) (width 0.2) (layer "F.Cu") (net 22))
 (segment (start 137.35 96.73) (end 137.35 97.24) (width 0.2) (layer "F.Cu") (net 22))
 (via (at 138.64 97.24) (size 0.25) (drill 0.4) (layers "F.Cu" "B.Cu") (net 22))
 (segment (start 136.4 98.42) (end 138.54 98.42) (width 0.2) (layer "B.Cu") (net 22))
 (segment (start 136.4 100.05) (end 136.4 98.42) (width 0.2) (layer "B.Cu") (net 22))
 (segment (start 138.64 98.32) (end 138.64 97.24) (width 0.2) (layer "B.Cu") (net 22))
 (segment (start 138.54 98.42) (end 138.61 98.35) (width 0.2) (layer "B.Cu") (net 22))
 (segment (start 138.61 98.35) (end 138.64 98.32) (width 0.2) (layer "B.Cu") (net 22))
 (segment (start 139.4 100.05) (end 139.4 99.3) (width 0.25) (layer "F.Cu") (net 16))
 (segment (start 139.4 99.3) (end 138.575489 98.475489) (width 0.25) (layer "F.Cu") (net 16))
 (segment (start 138.575489 98.475489) (end 137.305489 98.475489) (width 0.25) (layer "F.Cu") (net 16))
 (segment (start 136.365471 97.53096) (end 136.365471 97.535471) (width 0.25) (layer "F.Cu") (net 16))
 (segment (start 134.203632 97.53096) (end 136.365471 97.53096) (width 0.25) (layer "F.Cu") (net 16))
 (segment (start 136.365471 97.535471) (end 137.305489 98.475489) (width 0.25) (layer "F.Cu") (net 16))
 (segment (start 133.85 97.177328) (end 134.203632 97.53096) (width 0.25) (layer "F.Cu") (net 16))
 (segment (start 139.4 99.18) (end 139.4 100.05) (width 0.25) (layer "F.Cu") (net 16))
 (segment (start 133.85 96.73) (end 133.85 97.177328) (width 0.25) (layer "F.Cu") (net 16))
 (segment (start 138.05 94.53) (end 138.549022 94.53) (width 0.2) (layer "F.Cu") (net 26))
 (segment (start 139.04 95.020978) (end 138.549022 94.53) (width 0.2) (layer "F.Cu") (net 26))
 (segment (start 139.04 95.66) (end 139.04 95.020978) (width 0.2) (layer "F.Cu") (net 26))
 (via (at 139.04 95.66) (size 0.25) (drill 0.4) (layers "F.Cu" "B.Cu") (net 26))
 (segment (start 136.81048 96.88952) (end 137.81048 96.88952) (width 0.2) (layer "B.Cu") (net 26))
 (segment (start 134.4 100.05) (end 134.4 99.3) (width 0.2) (layer "B.Cu") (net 26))
 (segment (start 137.81048 96.88952) (end 139.04 95.66) (width 0.2) (layer "B.Cu") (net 26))
 (segment (start 134.4 99.3) (end 136.81048 96.88952) (width 0.2) (layer "B.Cu") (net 26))
 (segment (start 138.461973 90.53) (end 139.16 91.228027) (width 0.2) (layer "F.Cu") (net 34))
 (segment (start 138.05 90.53) (end 138.461973 90.53) (width 0.2) (layer "F.Cu") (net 34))
 (segment (start 139.16 91.228027) (end 139.16 93.5) (width 0.2) (layer "F.Cu") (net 34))
 (via (at 139.16 93.5) (size 0.25) (drill 0.4) (layers "F.Cu" "B.Cu") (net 34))
 (segment (start 139.16 94.67) (end 139.16 93.5) (width 0.2) (layer "B.Cu") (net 34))
 (segment (start 132.4 99.3) (end 133.45 98.25) (width 0.2) (layer "B.Cu") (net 34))
 (segment (start 137.34 96.49) (end 139.16 94.67) (width 0.2) (layer "B.Cu") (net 34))
 (segment (start 137.34 96.49) (end 136.19 96.49) (width 0.2) (layer "B.Cu") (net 34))
 (segment (start 136.19 96.49) (end 134.43 98.25) (width 0.2) (layer "B.Cu") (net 34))
 (segment (start 133.45 98.25) (end 134.43 98.25) (width 0.2) (layer "B.Cu") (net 34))
 (segment (start 132.4 100.05) (end 132.4 99.3) (width 0.2) (layer "B.Cu") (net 34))
 (segment (start 137.58 87.1) (end 138.99 87.1) (width 0.2) (layer "F.Cu") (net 36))
 (segment (start 138.99 87.1) (end 140.16548 88.27548) (width 0.2) (layer "F.Cu") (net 36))
 (segment (start 136.35 88.33) (end 137.58 87.1) (width 0.2) (layer "F.Cu") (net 36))
 (segment (start 136.35 89.83) (end 136.35 88.33) (width 0.2) (layer "F.Cu") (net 36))
 (segment (start 140.16548 96.41452) (end 139.82 96.76) (width 0.2) (layer "F.Cu") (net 36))
 (segment (start 140.16548 88.27548) (end 140.16548 96.41452) (width 0.2) (layer "F.Cu") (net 36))
 (via (at 139.82 96.76) (size 0.25) (drill 0.4) (layers "F.Cu" "B.Cu") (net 36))
 (segment (start 139.81 96.77) (end 139.82 96.76) (width 0.2) (layer "B.Cu") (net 36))
 (segment (start 138.4 100.05) (end 138.4 99.3) (width 0.2) (layer "B.Cu") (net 36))
 (segment (start 138.4 99.3) (end 139.81 97.89) (width 0.2) (layer "B.Cu") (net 36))
 (segment (start 139.81 97.89) (end 139.81 96.77) (width 0.2) (layer "B.Cu") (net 36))
 (segment (start 130.3 90.85) (end 130.49 91.04) (width 0.5) (layer "F.Cu") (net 4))
 (segment (start 131.15 87.72) (end 130.3 88.57) (width 0.5) (layer "F.Cu") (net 4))
 (segment (start 130.51 91.02) (end 130.49 91.04) (width 0.2) (layer "F.Cu") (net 4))
 (segment (start 131.15 91.03) (end 131.16 91.02) (width 0.2) (layer "F.Cu") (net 4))
 (segment (start 130.3 88.57) (end 130.3 90.85) (width 0.5) (layer "F.Cu") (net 4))
 (segment (start 131.15 85.25) (end 131.15 87.72) (width 0.5) (layer "F.Cu") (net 4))
 (segment (start 131.16 91.02) (end 130.51 91.02) (width 0.2) (layer "F.Cu") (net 4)))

